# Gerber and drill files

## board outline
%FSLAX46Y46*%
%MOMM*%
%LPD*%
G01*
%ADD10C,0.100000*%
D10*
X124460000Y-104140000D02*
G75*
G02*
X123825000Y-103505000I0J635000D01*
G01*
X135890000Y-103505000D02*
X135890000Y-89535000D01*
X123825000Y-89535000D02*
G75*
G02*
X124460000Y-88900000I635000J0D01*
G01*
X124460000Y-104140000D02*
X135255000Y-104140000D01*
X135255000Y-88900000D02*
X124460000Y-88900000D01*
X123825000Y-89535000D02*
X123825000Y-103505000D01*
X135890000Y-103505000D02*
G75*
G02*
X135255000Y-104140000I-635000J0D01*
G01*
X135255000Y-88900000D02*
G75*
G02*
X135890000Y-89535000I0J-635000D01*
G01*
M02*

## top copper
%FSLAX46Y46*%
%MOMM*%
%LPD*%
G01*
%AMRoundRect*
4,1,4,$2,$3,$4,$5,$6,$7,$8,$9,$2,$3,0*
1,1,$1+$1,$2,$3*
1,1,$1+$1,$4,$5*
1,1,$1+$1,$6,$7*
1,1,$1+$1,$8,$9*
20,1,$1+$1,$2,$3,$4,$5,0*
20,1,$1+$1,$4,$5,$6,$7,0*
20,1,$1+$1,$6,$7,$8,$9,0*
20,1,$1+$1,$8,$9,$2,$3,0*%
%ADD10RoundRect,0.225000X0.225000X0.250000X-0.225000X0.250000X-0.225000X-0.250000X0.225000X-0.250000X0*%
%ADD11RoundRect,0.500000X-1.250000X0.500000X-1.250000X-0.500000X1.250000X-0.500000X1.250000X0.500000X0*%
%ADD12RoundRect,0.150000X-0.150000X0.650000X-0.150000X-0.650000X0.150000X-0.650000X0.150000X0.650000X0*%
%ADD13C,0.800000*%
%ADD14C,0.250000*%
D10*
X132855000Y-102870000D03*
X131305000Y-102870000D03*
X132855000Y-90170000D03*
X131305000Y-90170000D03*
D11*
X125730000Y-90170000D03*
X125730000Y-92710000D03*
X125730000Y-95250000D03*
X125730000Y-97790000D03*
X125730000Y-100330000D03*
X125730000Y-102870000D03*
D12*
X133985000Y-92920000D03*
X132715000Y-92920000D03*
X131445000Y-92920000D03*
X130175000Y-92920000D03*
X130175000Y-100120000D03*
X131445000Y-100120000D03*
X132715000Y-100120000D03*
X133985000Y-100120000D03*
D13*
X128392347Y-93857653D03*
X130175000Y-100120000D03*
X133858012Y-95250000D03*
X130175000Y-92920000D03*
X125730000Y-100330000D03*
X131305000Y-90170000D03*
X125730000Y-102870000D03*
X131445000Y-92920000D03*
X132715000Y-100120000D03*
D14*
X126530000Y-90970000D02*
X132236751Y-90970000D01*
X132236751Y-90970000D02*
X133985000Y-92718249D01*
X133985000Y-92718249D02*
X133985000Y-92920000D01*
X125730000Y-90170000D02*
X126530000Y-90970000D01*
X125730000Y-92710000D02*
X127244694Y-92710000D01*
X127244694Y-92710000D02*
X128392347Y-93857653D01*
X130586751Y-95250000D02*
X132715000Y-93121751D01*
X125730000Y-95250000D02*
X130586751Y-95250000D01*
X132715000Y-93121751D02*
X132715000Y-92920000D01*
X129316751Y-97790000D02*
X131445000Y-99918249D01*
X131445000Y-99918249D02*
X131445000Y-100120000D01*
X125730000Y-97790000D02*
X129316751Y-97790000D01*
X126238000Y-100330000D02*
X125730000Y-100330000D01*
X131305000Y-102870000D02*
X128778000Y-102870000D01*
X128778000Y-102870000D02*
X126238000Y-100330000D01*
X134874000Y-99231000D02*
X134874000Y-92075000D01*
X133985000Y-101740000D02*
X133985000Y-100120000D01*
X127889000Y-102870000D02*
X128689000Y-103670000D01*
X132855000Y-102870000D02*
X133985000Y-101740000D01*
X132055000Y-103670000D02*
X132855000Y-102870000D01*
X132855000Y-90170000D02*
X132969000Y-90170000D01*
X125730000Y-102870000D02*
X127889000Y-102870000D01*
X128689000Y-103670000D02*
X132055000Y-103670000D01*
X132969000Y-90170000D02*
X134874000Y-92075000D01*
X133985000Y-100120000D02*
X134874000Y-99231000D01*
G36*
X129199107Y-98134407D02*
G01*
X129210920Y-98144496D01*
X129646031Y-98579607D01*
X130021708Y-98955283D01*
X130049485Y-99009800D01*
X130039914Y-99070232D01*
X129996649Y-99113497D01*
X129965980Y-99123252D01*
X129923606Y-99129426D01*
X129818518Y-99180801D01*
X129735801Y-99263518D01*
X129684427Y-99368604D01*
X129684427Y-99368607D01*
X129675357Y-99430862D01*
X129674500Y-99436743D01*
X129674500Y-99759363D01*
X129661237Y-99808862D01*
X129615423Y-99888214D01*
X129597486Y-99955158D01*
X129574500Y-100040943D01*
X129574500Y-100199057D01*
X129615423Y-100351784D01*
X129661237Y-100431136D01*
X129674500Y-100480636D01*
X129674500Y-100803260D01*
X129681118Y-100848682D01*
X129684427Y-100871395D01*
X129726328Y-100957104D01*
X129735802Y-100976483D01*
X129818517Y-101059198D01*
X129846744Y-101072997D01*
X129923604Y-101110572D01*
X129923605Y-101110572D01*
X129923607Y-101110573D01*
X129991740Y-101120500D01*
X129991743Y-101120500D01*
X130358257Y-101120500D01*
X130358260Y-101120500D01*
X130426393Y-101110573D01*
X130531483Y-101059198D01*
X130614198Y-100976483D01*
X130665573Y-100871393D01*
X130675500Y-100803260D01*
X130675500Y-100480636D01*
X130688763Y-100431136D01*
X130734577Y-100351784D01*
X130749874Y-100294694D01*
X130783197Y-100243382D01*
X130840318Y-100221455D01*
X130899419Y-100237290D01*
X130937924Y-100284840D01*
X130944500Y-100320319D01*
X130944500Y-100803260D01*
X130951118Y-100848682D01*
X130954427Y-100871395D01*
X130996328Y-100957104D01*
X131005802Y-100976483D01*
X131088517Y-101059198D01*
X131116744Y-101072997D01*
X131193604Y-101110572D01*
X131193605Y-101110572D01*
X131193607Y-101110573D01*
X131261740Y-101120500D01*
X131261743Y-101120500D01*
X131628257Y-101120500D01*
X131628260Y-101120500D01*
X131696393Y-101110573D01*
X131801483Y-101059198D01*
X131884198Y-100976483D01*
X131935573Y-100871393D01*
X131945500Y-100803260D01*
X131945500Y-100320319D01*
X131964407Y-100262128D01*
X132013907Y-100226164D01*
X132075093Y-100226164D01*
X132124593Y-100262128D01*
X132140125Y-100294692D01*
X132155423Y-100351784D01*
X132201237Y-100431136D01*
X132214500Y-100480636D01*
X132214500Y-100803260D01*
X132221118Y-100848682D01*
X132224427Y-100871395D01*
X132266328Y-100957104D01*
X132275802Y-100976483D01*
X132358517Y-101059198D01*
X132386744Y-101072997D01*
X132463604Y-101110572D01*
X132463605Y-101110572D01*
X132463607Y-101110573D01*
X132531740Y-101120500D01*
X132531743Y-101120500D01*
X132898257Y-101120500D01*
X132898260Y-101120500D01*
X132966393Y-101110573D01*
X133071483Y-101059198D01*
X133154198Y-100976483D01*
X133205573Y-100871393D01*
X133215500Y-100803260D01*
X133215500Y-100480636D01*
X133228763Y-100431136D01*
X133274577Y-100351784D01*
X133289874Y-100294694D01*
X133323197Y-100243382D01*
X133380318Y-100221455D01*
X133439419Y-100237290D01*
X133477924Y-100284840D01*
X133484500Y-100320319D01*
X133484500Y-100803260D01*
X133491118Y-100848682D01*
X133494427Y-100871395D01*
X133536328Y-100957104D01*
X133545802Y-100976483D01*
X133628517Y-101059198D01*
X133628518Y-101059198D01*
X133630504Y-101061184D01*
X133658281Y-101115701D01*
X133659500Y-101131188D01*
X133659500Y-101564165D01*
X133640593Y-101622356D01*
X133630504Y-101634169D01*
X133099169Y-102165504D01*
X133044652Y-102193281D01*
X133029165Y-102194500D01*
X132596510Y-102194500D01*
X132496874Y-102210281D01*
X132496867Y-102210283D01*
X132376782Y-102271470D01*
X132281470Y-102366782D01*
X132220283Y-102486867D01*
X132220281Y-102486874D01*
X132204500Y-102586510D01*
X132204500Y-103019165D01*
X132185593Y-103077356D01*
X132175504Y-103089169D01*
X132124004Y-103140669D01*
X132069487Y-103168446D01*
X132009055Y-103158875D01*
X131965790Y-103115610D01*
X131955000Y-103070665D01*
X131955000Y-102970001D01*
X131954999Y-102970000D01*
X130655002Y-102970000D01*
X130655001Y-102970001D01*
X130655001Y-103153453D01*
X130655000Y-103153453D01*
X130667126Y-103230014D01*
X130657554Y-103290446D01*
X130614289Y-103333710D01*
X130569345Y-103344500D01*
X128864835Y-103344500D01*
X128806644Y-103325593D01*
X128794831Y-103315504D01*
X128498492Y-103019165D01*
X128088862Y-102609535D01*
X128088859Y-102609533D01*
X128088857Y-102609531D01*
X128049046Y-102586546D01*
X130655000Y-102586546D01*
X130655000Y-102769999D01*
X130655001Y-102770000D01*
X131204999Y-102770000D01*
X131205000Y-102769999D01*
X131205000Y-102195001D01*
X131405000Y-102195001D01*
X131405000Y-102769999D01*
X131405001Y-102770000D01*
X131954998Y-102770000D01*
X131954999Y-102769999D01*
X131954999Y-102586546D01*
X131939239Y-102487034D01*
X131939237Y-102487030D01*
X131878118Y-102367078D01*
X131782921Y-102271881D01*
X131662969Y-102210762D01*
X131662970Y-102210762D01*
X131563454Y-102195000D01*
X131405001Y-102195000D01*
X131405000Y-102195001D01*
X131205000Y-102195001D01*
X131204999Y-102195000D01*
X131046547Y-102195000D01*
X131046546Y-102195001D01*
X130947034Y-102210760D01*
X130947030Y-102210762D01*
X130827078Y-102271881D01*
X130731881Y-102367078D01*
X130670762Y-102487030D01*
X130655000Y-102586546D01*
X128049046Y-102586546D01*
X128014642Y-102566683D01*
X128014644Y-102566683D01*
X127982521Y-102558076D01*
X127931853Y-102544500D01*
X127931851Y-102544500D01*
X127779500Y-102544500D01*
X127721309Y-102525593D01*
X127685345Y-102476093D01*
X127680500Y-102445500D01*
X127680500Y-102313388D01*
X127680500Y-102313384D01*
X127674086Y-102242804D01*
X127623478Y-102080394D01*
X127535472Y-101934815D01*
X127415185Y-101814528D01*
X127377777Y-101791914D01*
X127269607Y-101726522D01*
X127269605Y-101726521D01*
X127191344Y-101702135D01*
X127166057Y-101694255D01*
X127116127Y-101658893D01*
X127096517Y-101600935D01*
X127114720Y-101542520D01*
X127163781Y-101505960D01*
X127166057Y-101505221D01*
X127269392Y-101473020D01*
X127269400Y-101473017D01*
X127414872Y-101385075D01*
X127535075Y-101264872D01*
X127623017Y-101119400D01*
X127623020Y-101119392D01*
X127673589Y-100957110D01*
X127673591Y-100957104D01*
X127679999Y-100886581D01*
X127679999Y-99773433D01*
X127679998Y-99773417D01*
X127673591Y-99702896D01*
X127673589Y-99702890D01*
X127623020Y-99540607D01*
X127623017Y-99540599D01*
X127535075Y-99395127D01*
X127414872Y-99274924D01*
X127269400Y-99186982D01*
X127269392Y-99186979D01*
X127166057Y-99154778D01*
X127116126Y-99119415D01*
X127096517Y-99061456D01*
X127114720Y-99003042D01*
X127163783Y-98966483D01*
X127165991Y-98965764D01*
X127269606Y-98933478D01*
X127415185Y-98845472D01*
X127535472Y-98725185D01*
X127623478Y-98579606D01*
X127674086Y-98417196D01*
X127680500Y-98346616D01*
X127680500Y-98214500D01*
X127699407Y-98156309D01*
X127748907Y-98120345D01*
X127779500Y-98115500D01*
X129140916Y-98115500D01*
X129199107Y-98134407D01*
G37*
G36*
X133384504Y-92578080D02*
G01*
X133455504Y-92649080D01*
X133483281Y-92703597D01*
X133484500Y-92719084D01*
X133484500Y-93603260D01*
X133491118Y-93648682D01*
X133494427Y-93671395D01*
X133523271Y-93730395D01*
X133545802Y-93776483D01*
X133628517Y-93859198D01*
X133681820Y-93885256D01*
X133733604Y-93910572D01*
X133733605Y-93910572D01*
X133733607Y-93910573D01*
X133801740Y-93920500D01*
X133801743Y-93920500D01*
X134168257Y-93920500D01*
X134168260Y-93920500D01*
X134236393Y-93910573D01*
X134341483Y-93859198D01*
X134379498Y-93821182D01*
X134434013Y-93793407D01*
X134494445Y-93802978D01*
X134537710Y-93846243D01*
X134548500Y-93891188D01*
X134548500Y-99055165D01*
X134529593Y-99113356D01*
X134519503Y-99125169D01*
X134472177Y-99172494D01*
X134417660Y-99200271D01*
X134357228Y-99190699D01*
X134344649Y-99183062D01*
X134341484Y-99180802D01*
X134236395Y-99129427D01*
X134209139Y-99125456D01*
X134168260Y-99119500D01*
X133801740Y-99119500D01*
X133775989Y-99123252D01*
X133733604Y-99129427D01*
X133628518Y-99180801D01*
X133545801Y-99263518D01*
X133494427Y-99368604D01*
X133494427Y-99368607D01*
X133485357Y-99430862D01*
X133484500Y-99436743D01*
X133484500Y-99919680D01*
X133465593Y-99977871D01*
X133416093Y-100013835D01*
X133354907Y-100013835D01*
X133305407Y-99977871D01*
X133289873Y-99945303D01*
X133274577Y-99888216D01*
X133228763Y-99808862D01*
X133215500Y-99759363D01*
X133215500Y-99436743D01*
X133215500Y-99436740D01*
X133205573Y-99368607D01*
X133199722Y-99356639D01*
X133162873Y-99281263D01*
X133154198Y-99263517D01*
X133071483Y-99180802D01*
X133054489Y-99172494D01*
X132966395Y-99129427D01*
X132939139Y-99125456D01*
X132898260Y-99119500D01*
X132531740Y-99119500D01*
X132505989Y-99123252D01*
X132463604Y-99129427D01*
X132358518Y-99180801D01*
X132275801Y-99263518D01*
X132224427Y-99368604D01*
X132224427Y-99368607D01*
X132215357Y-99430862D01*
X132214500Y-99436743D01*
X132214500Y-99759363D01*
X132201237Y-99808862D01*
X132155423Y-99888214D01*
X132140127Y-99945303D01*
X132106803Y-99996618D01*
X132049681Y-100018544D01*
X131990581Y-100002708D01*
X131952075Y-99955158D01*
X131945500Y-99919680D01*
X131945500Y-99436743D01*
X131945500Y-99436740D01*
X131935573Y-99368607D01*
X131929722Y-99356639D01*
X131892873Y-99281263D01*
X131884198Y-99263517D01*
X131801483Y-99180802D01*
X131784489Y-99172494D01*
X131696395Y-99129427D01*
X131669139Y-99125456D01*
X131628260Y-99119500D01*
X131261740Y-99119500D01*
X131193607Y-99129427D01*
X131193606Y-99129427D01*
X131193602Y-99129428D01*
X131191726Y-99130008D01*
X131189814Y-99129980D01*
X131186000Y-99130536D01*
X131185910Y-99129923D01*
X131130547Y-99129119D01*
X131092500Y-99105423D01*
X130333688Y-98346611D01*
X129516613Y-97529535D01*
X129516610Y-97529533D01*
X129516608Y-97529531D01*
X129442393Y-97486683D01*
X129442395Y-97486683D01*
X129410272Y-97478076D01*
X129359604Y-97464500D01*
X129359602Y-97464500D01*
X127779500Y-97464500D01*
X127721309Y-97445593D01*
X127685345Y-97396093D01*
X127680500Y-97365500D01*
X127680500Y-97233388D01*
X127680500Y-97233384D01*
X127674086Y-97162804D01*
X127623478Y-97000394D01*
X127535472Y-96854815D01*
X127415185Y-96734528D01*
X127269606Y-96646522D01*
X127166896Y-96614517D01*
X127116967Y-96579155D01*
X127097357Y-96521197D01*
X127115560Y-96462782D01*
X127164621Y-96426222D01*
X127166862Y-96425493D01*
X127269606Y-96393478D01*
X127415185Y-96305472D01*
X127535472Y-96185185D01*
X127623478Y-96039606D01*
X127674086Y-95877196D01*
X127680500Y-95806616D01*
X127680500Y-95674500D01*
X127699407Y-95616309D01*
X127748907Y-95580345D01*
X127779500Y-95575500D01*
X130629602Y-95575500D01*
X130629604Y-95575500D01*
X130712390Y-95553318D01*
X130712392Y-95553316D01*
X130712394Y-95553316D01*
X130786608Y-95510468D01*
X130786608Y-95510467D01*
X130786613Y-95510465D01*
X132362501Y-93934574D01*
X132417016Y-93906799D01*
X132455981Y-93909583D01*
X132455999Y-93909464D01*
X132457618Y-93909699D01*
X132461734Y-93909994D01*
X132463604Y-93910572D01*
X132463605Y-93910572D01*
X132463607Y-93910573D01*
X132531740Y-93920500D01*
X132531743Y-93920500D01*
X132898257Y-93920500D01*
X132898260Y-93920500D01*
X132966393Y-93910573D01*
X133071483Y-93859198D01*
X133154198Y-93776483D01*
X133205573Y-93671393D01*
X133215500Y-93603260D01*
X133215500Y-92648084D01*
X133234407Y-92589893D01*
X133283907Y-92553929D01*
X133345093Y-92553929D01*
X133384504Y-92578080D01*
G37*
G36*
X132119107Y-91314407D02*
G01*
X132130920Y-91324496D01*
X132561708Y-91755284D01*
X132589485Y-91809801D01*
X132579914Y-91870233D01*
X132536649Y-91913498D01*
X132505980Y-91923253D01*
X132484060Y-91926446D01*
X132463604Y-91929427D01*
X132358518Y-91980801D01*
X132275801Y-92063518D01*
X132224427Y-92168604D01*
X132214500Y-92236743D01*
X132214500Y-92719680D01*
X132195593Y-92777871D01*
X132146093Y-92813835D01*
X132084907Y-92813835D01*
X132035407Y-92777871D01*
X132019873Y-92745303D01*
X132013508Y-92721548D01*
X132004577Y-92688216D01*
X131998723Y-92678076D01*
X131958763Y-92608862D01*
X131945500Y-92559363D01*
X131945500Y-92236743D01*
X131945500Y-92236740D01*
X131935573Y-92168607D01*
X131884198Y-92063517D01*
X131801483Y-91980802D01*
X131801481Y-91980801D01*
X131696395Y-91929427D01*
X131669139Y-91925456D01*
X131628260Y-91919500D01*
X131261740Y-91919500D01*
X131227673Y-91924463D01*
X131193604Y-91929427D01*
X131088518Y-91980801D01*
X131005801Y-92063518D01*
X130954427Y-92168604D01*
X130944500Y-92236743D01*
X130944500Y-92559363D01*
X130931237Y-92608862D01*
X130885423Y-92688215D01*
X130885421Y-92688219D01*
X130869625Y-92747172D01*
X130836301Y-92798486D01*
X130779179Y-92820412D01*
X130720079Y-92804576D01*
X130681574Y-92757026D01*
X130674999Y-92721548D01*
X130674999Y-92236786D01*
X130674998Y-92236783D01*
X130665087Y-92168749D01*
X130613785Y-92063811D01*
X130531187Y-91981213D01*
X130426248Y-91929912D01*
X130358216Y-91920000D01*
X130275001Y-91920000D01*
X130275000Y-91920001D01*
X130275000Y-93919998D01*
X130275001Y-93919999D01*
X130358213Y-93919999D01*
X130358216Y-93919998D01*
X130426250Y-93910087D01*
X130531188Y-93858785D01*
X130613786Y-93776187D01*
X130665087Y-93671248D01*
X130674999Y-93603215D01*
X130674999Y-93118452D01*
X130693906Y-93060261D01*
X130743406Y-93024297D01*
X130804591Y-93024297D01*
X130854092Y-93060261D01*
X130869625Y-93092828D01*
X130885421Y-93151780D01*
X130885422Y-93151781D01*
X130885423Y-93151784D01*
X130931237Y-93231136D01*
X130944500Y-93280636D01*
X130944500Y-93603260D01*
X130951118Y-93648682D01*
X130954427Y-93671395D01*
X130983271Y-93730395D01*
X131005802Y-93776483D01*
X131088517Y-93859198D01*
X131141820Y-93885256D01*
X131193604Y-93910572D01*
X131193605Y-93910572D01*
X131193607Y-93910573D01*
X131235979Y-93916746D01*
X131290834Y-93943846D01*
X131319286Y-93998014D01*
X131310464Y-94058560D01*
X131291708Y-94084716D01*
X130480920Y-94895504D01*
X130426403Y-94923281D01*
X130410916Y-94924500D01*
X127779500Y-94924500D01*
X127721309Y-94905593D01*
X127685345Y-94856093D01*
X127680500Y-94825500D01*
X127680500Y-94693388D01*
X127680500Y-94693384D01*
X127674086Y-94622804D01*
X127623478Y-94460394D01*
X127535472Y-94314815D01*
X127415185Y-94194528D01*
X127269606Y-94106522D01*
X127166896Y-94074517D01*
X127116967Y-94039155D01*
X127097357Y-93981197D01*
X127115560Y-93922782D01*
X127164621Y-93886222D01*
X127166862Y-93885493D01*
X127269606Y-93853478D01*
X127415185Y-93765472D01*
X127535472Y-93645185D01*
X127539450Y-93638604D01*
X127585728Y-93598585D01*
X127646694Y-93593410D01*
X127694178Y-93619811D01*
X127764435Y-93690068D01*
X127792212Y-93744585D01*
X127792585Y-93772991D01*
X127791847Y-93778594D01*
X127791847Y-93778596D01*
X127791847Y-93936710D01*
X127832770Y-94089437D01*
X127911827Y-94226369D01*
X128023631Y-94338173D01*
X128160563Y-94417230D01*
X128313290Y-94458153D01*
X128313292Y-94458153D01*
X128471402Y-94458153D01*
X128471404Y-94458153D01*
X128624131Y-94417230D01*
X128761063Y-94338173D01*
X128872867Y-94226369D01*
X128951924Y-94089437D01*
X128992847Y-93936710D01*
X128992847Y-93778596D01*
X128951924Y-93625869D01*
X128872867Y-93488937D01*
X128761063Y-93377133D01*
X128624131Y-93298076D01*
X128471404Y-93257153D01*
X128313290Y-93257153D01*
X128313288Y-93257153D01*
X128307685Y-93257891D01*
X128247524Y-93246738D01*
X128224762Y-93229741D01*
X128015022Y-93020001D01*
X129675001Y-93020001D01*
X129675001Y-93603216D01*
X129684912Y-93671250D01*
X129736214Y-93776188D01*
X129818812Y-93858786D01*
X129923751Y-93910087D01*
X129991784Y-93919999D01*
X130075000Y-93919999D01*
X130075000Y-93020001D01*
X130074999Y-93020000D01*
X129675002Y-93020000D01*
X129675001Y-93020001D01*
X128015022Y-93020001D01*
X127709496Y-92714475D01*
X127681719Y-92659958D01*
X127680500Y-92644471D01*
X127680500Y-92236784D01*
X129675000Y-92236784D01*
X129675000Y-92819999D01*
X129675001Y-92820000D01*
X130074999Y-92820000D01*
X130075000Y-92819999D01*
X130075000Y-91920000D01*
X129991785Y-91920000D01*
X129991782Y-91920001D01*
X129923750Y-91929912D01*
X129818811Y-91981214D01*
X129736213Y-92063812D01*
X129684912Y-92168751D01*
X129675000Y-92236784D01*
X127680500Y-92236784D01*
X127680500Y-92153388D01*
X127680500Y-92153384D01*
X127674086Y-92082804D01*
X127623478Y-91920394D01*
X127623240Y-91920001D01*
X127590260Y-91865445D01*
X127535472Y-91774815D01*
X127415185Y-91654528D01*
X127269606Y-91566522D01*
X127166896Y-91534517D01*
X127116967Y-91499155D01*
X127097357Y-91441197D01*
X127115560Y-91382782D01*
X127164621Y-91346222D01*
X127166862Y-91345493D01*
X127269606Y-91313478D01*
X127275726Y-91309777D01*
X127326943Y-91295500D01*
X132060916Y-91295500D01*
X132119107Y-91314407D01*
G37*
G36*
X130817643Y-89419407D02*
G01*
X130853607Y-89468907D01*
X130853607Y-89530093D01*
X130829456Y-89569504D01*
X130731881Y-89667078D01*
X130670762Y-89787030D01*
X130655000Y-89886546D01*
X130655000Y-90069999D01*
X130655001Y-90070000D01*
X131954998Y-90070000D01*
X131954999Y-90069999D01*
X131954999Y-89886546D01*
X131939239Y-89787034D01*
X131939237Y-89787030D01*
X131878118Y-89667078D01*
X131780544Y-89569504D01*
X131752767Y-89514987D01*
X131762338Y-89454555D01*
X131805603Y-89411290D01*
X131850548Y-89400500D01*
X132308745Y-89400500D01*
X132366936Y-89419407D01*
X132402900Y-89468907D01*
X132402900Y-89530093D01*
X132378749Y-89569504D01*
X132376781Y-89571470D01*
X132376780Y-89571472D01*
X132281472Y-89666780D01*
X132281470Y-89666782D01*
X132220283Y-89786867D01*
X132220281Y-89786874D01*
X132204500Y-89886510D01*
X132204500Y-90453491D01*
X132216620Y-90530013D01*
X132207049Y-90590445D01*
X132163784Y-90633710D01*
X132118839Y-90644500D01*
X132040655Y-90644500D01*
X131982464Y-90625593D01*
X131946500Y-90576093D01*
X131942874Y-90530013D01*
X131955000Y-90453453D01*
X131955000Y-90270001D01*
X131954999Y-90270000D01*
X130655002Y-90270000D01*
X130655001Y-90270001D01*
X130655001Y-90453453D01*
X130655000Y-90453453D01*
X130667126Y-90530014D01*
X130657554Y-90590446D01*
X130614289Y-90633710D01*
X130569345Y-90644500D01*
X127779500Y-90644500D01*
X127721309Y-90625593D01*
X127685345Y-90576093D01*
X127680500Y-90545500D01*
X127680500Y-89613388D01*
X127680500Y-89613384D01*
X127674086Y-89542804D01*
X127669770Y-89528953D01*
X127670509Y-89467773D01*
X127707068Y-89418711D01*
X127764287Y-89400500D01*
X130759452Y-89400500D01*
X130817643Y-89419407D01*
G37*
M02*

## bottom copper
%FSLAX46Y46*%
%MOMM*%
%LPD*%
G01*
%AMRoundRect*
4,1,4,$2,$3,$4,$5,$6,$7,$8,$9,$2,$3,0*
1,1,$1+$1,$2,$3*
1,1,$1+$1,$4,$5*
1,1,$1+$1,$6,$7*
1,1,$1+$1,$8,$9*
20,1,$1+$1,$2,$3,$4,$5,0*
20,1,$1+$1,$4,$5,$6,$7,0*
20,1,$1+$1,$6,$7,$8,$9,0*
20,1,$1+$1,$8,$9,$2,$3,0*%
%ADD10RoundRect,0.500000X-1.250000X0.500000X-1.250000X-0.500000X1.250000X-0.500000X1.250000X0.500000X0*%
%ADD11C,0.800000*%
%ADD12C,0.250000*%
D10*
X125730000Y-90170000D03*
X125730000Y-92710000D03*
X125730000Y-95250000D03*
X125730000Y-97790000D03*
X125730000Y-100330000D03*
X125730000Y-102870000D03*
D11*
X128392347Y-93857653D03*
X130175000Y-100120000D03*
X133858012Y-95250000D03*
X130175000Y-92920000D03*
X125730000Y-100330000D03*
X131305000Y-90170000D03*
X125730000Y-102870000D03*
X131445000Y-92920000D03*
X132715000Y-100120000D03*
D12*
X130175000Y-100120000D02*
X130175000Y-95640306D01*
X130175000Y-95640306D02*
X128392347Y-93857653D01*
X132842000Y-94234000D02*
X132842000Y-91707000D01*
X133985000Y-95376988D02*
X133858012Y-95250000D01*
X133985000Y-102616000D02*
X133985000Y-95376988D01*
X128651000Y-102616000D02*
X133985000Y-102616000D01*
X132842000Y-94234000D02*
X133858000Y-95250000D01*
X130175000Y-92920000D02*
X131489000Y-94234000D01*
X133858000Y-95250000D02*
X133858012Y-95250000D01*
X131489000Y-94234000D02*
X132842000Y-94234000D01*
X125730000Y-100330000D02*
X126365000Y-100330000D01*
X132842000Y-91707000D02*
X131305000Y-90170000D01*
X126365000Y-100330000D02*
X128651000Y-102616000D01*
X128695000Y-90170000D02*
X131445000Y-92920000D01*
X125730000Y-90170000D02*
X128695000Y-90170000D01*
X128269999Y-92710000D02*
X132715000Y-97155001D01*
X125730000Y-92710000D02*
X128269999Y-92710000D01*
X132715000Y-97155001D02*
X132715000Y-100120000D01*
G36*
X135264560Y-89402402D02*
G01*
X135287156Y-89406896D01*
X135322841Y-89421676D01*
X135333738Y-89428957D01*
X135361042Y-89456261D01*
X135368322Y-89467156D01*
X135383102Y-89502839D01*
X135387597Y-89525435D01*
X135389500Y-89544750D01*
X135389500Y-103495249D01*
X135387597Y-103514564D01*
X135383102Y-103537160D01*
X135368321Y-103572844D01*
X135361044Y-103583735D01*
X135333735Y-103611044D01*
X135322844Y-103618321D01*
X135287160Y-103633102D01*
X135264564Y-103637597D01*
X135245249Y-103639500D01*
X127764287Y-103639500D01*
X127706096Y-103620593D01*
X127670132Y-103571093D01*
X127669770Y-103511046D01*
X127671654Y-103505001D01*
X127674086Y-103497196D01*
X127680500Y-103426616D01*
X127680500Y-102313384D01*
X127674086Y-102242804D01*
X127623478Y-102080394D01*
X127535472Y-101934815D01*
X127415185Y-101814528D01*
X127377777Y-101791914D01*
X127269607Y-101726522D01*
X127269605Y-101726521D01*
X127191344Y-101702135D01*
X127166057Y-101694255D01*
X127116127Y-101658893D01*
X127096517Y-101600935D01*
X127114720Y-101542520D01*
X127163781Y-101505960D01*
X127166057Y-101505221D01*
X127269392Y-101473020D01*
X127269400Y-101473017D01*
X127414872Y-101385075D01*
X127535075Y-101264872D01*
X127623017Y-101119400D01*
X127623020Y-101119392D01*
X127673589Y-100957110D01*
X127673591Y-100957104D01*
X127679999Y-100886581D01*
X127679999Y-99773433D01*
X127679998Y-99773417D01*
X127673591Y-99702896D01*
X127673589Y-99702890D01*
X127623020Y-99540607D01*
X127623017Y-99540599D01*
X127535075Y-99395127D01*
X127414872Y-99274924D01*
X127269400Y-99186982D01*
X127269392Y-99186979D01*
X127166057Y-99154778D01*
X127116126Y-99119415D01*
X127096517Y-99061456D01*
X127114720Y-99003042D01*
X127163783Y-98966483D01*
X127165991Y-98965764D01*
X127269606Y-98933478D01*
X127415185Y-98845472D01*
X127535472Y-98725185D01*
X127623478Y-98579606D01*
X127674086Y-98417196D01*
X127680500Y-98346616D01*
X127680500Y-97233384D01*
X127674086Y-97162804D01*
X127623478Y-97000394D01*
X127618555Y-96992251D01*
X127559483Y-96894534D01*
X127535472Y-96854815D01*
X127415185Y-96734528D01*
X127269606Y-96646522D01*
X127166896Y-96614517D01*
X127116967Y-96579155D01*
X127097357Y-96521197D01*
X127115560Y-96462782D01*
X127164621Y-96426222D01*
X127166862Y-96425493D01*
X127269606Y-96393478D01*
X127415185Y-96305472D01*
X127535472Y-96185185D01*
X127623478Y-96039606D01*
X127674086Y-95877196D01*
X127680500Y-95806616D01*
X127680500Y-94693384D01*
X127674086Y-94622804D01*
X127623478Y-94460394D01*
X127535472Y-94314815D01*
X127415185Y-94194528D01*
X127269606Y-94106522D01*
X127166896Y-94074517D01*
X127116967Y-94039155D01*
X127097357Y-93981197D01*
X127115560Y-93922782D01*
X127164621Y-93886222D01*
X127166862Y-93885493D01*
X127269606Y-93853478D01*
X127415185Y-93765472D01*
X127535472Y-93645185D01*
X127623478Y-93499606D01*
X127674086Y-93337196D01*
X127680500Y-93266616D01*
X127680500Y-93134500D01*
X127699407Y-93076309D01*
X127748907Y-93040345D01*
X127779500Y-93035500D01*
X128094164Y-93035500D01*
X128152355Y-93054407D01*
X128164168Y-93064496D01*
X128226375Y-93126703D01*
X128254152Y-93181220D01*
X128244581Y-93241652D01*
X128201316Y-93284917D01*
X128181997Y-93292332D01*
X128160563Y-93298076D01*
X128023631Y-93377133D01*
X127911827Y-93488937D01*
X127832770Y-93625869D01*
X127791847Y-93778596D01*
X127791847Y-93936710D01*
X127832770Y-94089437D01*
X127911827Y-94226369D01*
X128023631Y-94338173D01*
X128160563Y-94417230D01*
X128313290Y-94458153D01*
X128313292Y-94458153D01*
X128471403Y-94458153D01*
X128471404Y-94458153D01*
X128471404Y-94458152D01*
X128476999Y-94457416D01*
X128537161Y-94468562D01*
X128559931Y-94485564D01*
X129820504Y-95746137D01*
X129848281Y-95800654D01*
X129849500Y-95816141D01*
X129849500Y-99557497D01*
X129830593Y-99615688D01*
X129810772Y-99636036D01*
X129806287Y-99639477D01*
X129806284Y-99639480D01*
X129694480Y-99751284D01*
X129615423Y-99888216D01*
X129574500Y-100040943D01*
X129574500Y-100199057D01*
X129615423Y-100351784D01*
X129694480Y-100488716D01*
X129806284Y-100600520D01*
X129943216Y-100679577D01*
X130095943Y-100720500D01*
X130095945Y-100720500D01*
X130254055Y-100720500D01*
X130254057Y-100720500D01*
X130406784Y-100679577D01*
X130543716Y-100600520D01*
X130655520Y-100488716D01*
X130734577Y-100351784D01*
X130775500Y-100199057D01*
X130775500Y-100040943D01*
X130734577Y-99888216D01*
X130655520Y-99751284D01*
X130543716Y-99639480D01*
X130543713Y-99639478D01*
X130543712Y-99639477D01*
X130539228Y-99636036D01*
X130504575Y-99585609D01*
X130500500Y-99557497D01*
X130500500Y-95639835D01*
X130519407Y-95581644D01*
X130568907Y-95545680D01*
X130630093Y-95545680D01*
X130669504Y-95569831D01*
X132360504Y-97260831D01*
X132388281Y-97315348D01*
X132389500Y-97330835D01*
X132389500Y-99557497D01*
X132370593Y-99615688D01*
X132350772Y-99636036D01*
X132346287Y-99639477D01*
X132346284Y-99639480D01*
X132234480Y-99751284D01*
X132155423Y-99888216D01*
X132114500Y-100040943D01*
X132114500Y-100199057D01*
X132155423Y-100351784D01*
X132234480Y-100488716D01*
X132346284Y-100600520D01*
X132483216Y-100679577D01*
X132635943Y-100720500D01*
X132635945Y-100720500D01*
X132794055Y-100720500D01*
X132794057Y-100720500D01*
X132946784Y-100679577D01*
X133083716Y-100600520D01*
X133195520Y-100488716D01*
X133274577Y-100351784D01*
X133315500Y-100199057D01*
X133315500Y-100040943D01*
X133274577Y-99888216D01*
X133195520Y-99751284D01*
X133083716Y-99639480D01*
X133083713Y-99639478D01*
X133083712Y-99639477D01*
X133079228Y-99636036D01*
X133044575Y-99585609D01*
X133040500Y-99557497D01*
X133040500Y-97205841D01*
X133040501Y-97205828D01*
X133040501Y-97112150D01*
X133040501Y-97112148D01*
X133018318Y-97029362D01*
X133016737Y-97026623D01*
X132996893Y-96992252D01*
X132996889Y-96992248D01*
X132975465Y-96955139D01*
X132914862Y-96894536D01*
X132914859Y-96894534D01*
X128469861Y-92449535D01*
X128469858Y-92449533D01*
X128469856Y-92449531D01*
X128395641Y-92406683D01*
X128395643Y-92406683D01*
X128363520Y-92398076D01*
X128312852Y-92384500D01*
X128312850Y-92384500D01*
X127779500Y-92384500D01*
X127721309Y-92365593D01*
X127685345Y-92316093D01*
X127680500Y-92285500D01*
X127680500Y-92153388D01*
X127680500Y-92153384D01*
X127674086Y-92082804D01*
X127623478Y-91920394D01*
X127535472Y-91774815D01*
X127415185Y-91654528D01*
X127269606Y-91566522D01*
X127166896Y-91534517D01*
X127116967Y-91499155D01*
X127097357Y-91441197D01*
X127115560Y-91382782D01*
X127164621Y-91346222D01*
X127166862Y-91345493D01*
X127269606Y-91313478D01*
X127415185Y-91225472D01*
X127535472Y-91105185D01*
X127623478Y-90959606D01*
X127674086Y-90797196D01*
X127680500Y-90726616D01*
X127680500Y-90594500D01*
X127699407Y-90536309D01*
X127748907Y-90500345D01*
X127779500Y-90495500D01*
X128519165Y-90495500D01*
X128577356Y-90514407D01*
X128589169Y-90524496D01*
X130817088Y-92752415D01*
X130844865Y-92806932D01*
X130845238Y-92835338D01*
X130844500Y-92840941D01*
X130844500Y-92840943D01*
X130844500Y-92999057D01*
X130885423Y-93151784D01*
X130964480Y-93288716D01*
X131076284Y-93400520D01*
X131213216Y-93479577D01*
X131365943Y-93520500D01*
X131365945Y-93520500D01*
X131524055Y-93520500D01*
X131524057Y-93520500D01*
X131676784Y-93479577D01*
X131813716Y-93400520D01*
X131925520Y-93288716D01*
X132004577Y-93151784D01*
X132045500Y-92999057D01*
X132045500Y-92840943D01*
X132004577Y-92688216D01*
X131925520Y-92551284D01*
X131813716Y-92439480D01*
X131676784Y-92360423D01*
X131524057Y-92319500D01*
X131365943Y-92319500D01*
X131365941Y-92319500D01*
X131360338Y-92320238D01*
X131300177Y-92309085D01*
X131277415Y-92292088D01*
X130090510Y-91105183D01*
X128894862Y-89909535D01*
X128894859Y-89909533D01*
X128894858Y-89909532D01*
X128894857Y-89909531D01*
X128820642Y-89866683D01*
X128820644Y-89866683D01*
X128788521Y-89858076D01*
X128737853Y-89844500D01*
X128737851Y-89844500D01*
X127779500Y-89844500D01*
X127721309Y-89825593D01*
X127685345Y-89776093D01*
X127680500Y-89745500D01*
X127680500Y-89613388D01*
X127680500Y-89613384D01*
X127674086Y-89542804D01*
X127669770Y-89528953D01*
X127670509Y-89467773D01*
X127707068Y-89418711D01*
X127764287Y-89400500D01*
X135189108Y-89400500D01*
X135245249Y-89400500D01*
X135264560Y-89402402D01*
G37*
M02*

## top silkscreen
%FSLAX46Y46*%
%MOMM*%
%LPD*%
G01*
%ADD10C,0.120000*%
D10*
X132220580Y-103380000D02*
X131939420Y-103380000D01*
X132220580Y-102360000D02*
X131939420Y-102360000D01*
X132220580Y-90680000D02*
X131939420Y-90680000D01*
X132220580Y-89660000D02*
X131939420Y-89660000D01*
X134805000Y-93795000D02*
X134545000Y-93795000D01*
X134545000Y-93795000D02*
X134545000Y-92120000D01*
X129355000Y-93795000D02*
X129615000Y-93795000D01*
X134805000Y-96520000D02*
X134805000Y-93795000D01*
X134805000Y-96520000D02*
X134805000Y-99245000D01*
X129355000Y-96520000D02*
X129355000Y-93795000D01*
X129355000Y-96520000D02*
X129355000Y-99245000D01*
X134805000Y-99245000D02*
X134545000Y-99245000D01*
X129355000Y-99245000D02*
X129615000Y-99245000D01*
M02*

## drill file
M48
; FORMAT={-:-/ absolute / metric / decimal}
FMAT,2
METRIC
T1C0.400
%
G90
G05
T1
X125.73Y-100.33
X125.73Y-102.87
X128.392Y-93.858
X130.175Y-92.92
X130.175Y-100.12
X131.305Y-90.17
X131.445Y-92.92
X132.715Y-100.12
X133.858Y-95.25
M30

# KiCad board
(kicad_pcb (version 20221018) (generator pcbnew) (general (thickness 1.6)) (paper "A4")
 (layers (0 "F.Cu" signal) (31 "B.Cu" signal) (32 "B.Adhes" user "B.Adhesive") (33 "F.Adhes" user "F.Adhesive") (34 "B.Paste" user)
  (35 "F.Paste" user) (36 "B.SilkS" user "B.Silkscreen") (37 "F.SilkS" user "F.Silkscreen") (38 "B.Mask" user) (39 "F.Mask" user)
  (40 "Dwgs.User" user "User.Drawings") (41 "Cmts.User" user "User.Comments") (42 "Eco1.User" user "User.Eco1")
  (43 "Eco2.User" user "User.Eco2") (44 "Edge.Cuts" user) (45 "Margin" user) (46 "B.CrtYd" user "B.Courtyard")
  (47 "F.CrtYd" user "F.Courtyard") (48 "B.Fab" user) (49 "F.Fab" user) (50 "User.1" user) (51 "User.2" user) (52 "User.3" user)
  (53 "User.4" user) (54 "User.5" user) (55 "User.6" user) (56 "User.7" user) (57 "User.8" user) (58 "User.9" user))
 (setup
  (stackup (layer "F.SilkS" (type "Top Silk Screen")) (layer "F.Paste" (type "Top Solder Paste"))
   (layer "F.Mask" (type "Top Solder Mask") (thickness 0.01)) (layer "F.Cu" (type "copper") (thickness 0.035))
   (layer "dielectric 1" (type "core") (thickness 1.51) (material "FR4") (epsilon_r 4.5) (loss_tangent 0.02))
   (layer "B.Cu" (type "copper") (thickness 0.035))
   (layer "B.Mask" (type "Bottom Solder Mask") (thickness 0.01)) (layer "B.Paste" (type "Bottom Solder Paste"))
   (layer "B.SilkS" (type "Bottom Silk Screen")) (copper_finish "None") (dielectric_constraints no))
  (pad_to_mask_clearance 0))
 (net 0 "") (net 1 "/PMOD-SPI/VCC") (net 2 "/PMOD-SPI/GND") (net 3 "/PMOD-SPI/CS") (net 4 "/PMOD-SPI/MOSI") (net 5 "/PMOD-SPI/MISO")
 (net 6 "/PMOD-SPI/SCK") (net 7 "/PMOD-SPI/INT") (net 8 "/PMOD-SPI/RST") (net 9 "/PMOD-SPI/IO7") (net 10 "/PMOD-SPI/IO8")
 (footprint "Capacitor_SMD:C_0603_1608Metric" (layer "F.Cu") (at 132.08 102.87 180)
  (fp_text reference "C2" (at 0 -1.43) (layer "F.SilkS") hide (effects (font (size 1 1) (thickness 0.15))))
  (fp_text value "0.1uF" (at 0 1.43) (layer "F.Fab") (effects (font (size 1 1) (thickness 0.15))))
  (fp_line (start -0.14058 -0.51) (end 0.14058 -0.51) (stroke (width 0.12) (type solid)) (layer "F.SilkS"))
  (fp_line (start -0.14058 0.51) (end 0.14058 0.51) (stroke (width 0.12) (type solid)) (layer "F.SilkS"))
  (pad "1" smd roundrect (at -0.775 0 180) (size 0.9 0.95) (layers "F.Cu" "F.Paste" "F.Mask") (roundrect_rratio 0.25)
   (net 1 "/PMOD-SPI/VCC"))
  (pad "2" smd roundrect (at 0.775 0 180) (size 0.9 0.95) (layers "F.Cu" "F.Paste" "F.Mask") (roundrect_rratio 0.25) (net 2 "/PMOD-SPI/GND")))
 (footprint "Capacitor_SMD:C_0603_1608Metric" (layer "F.Cu") (at 132.08 90.17 180)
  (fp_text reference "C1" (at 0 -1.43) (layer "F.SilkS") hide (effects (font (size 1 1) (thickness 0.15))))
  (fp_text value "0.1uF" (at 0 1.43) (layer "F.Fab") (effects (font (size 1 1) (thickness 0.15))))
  (fp_line (start -0.14058 -0.51) (end 0.14058 -0.51) (stroke (width 0.12) (type solid)) (layer "F.SilkS"))
  (fp_line (start -0.14058 0.51) (end 0.14058 0.51) (stroke (width 0.12) (type solid)) (layer "F.SilkS"))
  (pad "1" smd roundrect (at -0.775 0 180) (size 0.9 0.95) (layers "F.Cu" "F.Paste" "F.Mask") (roundrect_rratio 0.25)
   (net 1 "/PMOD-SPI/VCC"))
  (pad "2" smd roundrect (at 0.775 0 180) (size 0.9 0.95) (layers "F.Cu" "F.Paste" "F.Mask") (roundrect_rratio 0.25) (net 2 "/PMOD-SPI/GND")))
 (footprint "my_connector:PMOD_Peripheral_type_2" (layer "F.Cu") (at 125.73 96.52 -90)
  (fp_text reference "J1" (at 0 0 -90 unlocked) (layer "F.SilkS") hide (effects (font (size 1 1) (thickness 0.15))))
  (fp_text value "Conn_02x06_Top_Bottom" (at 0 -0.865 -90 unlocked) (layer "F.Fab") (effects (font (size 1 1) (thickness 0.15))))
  (pad "1" smd roundrect (at -6.35 0 270) (size 2 3.5) (layers "F.Cu" "F.Paste" "F.Mask") (roundrect_rratio 0.25) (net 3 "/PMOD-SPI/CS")
   (thermal_bridge_angle 45))
  (pad "2" smd roundrect (at -3.81 0 270) (size 2 3.5) (layers "F.Cu" "F.Paste" "F.Mask") (roundrect_rratio 0.25) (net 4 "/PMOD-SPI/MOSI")
   (thermal_bridge_angle 45))
  (pad "3" smd roundrect (at -1.27 0 270) (size 2 3.5) (layers "F.Cu" "F.Paste" "F.Mask") (roundrect_rratio 0.25) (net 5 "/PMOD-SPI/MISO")
   (thermal_bridge_angle 45))
  (pad "4" smd roundrect (at 1.27 0 270) (size 2 3.5) (layers "F.Cu" "F.Paste" "F.Mask") (roundrect_rratio 0.25) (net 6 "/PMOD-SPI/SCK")
   (thermal_bridge_angle 45))
  (pad "5" smd roundrect (at 3.81 0 270) (size 2 3.5) (layers "F.Cu" "F.Paste" "F.Mask") (roundrect_rratio 0.25) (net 2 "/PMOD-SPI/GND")
   (thermal_bridge_angle 45))
  (pad "6" smd roundrect (at 6.35 0 270) (size 2 3.5) (layers "F.Cu" "F.Paste" "F.Mask") (roundrect_rratio 0.25) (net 1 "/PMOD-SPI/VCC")
   (thermal_bridge_angle 45))
  (pad "7" smd roundrect (at -6.35 0 270) (size 2 3.5) (layers "B.Cu" "B.Paste" "B.Mask") (roundrect_rratio 0.25) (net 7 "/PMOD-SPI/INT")
   (thermal_bridge_angle 45))
  (pad "8" smd roundrect (at -3.81 0 270) (size 2 3.5) (layers "B.Cu" "B.Paste" "B.Mask") (roundrect_rratio 0.25) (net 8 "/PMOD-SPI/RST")
   (thermal_bridge_angle 45))
  (pad "9" smd roundrect (at -1.27 0 270) (size 2 3.5) (layers "B.Cu" "B.Paste" "B.Mask") (roundrect_rratio 0.25) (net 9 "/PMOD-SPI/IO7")
   (thermal_bridge_angle 45))
  (pad "10" smd roundrect (at 1.27 0 270) (size 2 3.5) (layers "B.Cu" "B.Paste" "B.Mask") (roundrect_rratio 0.25) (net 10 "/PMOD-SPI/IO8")
   (thermal_bridge_angle 45))
  (pad "11" smd roundrect (at 3.81 0 270) (size 2 3.5) (layers "B.Cu" "B.Paste" "B.Mask") (roundrect_rratio 0.25) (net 2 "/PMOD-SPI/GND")
   (thermal_bridge_angle 45))
  (pad "12" smd roundrect (at 6.35 0 270) (size 2 3.5) (layers "B.Cu" "B.Paste" "B.Mask") (roundrect_rratio 0.25) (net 1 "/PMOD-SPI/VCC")
   (thermal_bridge_angle 45)))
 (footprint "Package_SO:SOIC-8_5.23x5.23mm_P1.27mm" (layer "F.Cu") (at 132.08 96.52 -90)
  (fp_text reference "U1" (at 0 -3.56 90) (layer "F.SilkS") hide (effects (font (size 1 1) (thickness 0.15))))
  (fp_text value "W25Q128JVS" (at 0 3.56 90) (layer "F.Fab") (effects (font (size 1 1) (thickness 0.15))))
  (fp_line (start -2.725 -2.725) (end -2.725 -2.465) (stroke (width 0.12) (type solid)) (layer "F.SilkS"))
  (fp_line (start -2.725 -2.465) (end -4.4 -2.465) (stroke (width 0.12) (type solid)) (layer "F.SilkS"))
  (fp_line (start -2.725 2.725) (end -2.725 2.465) (stroke (width 0.12) (type solid)) (layer "F.SilkS"))
  (fp_line (start 0 -2.725) (end -2.725 -2.725) (stroke (width 0.12) (type solid)) (layer "F.SilkS"))
  (fp_line (start 0 -2.725) (end 2.725 -2.725) (stroke (width 0.12) (type solid)) (layer "F.SilkS"))
  (fp_line (start 0 2.725) (end -2.725 2.725) (stroke (width 0.12) (type solid)) (layer "F.SilkS"))
  (fp_line (start 0 2.725) (end 2.725 2.725) (stroke (width 0.12) (type solid)) (layer "F.SilkS"))
  (fp_line (start 2.725 -2.725) (end 2.725 -2.465) (stroke (width 0.12) (type solid)) (layer "F.SilkS"))
  (fp_line (start 2.725 2.725) (end 2.725 2.465) (stroke (width 0.12) (type solid)) (layer "F.SilkS"))
  (pad "1" smd roundrect (at -3.6 -1.905 270) (size 1.6 0.6) (layers "F.Cu" "F.Paste" "F.Mask") (roundrect_rratio 0.25)
   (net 3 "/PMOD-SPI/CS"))
  (pad "2" smd roundrect (at -3.6 -0.635 270) (size 1.6 0.6) (layers "F.Cu" "F.Paste" "F.Mask") (roundrect_rratio 0.25)
   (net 5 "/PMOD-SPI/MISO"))
  (pad "3" smd roundrect (at -3.6 0.635 270) (size 1.6 0.6) (layers "F.Cu" "F.Paste" "F.Mask") (roundrect_rratio 0.25)
   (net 7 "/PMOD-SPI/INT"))
  (pad "4" smd roundrect (at -3.6 1.905 270) (size 1.6 0.6) (layers "F.Cu" "F.Paste" "F.Mask") (roundrect_rratio 0.25)
   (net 2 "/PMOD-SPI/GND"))
  (pad "5" smd roundrect (at 3.6 1.905 270) (size 1.6 0.6) (layers "F.Cu" "F.Paste" "F.Mask") (roundrect_rratio 0.25)
   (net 4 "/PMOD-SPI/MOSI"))
  (pad "6" smd roundrect (at 3.6 0.635 270) (size 1.6 0.6) (layers "F.Cu" "F.Paste" "F.Mask") (roundrect_rratio 0.25)
   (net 6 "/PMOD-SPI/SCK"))
  (pad "7" smd roundrect (at 3.6 -0.635 270) (size 1.6 0.6) (layers "F.Cu" "F.Paste" "F.Mask") (roundrect_rratio 0.25)
   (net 8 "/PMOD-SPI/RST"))
  (pad "8" smd roundrect (at 3.6 -1.905 270) (size 1.6 0.6) (layers "F.Cu" "F.Paste" "F.Mask") (roundrect_rratio 0.25)
   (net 1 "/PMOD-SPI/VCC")))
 (gr_arc (start 124.46 104.14) (mid 124.010987 103.954013) (end 123.825 103.505) (stroke (width 0.1) (type default)) (layer "Edge.Cuts"))
 (gr_line (start 135.89 103.505) (end 135.89 89.535) (stroke (width 0.1) (type default)) (layer "Edge.Cuts"))
 (gr_arc (start 123.825 89.535) (mid 124.010987 89.085987) (end 124.46 88.9) (stroke (width 0.1) (type default)) (layer "Edge.Cuts"))
 (gr_line (start 124.46 104.14) (end 135.255 104.14) (stroke (width 0.1) (type default)) (layer "Edge.Cuts"))
 (gr_line (start 135.255 88.9) (end 124.46 88.9) (stroke (width 0.1) (type default)) (layer "Edge.Cuts"))
 (gr_line (start 123.825 89.535) (end 123.825 103.505) (stroke (width 0.1) (type default)) (layer "Edge.Cuts"))
 (gr_arc (start 135.89 103.505) (mid 135.704013 103.954013) (end 135.255 104.14) (stroke (width 0.1) (type default)) (layer "Edge.Cuts"))
 (gr_arc (start 135.255 88.9) (mid 135.704013 89.085987) (end 135.89 89.535) (stroke (width 0.1) (type default)) (layer "Edge.Cuts"))
 (segment (start 126.53 90.97) (end 132.236751 90.97) (width 0.25) (layer "F.Cu") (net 3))
 (segment (start 132.236751 90.97) (end 133.985 92.718249) (width 0.25) (layer "F.Cu") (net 3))
 (segment (start 133.985 92.718249) (end 133.985 92.92) (width 0.25) (layer "F.Cu") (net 3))
 (segment (start 125.73 90.17) (end 126.53 90.97) (width 0.25) (layer "F.Cu") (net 3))
 (segment (start 125.73 92.71) (end 127.244694 92.71) (width 0.25) (layer "F.Cu") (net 4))
 (segment (start 127.244694 92.71) (end 128.392347 93.857653) (width 0.25) (layer "F.Cu") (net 4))
 (via (at 128.392347 93.857653) (size 0.8) (drill 0.4) (layers "F.Cu" "B.Cu") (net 4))
 (via (at 130.175 100.12) (size 0.8) (drill 0.4) (layers "F.Cu" "B.Cu") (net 4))
 (segment (start 130.175 100.12) (end 130.175 95.640306) (width 0.25) (layer "B.Cu") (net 4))
 (segment (start 130.175 95.640306) (end 128.392347 93.857653) (width 0.25) (layer "B.Cu") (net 4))
 (segment (start 130.586751 95.25) (end 132.715 93.121751) (width 0.25) (layer "F.Cu") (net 5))
 (segment (start 125.73 95.25) (end 130.586751 95.25) (width 0.25) (layer "F.Cu") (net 5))
 (segment (start 132.715 93.121751) (end 132.715 92.92) (width 0.25) (layer "F.Cu") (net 5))
 (segment (start 129.316751 97.79) (end 131.445 99.918249) (width 0.25) (layer "F.Cu") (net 6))
 (segment (start 131.445 99.918249) (end 131.445 100.12) (width 0.25) (layer "F.Cu") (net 6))
 (segment (start 125.73 97.79) (end 129.316751 97.79) (width 0.25) (layer "F.Cu") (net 6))
 (segment (start 126.238 100.33) (end 125.73 100.33) (width 0.25) (layer "F.Cu") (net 2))
 (segment (start 131.305 102.87) (end 128.778 102.87) (width 0.25) (layer "F.Cu") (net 2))
 (segment (start 128.778 102.87) (end 126.238 100.33) (width 0.25) (layer "F.Cu") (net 2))
 (via (at 133.858012 95.25) (size 0.8) (drill 0.4) (layers "F.Cu" "B.Cu") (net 2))
 (via (at 130.175 92.92) (size 0.8) (drill 0.4) (layers "F.Cu" "B.Cu") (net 2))
 (via (at 125.73 100.33) (size 0.8) (drill 0.4) (layers "F.Cu" "B.Cu") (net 2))
 (via (at 131.305 90.17) (size 0.8) (drill 0.4) (layers "F.Cu" "B.Cu") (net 2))
 (segment (start 132.842 94.234) (end 132.842 91.707) (width 0.25) (layer "B.Cu") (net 2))
 (segment (start 133.985 95.376988) (end 133.858012 95.25) (width 0.25) (layer "B.Cu") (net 2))
 (segment (start 133.985 102.616) (end 133.985 95.376988) (width 0.25) (layer "B.Cu") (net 2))
 (segment (start 128.651 102.616) (end 133.985 102.616) (width 0.25) (layer "B.Cu") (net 2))
 (segment (start 132.842 94.234) (end 133.858 95.25) (width 0.25) (layer "B.Cu") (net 2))
 (segment (start 130.175 92.92) (end 131.489 94.234) (width 0.25) (layer "B.Cu") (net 2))
 (segment (start 133.858 95.25) (end 133.858012 95.25) (width 0.25) (layer "B.Cu") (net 2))
 (segment (start 131.489 94.234) (end 132.842 94.234) (width 0.25) (layer "B.Cu") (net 2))
 (segment (start 125.73 100.33) (end 126.365 100.33) (width 0.25) (layer "B.Cu") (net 2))
 (segment (start 132.842 91.707) (end 131.305 90.17) (width 0.25) (layer "B.Cu") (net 2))
 (segment (start 126.365 100.33) (end 128.651 102.616) (width 0.25) (layer "B.Cu") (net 2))
 (segment (start 134.874 99.231) (end 134.874 92.075) (width 0.25) (layer "F.Cu") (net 1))
 (segment (start 133.985 101.74) (end 133.985 100.12) (width 0.25) (layer "F.Cu") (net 1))
 (segment (start 127.889 102.87) (end 128.689 103.67) (width 0.25) (layer "F.Cu") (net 1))
 (segment (start 132.855 102.87) (end 133.985 101.74) (width 0.25) (layer "F.Cu") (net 1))
 (segment (start 132.055 103.67) (end 132.855 102.87) (width 0.25) (layer "F.Cu") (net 1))
 (segment (start 132.855 90.17) (end 132.969 90.17) (width 0.25) (layer "F.Cu") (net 1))
 (segment (start 125.73 102.87) (end 127.889 102.87) (width 0.25) (layer "F.Cu") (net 1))
 (segment (start 128.689 103.67) (end 132.055 103.67) (width 0.25) (layer "F.Cu") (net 1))
 (segment (start 132.969 90.17) (end 134.874 92.075) (width 0.25) (layer "F.Cu") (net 1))
 (segment (start 133.985 100.12) (end 134.874 99.231) (width 0.25) (layer "F.Cu") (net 1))
 (via (at 125.73 102.87) (size 0.8) (drill 0.4) (layers "F.Cu" "B.Cu") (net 1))
 (via (at 131.445 92.92) (size 0.8) (drill 0.4) (layers "F.Cu" "B.Cu") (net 7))
 (segment (start 128.695 90.17) (end 131.445 92.92) (width 0.25) (layer "B.Cu") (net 7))
 (segment (start 125.73 90.17) (end 128.695 90.17) (width 0.25) (layer "B.Cu") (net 7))
 (via (at 132.715 100.12) (size 0.8) (drill 0.4) (layers "F.Cu" "B.Cu") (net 8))
 (segment (start 128.269999 92.71) (end 132.715 97.155001) (width 0.25) (layer "B.Cu") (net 8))
 (segment (start 125.73 92.71) (end 128.269999 92.71) (width 0.25) (layer "B.Cu") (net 8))
 (segment (start 132.715 97.155001) (end 132.715 100.12) (width 0.25) (layer "B.Cu") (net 8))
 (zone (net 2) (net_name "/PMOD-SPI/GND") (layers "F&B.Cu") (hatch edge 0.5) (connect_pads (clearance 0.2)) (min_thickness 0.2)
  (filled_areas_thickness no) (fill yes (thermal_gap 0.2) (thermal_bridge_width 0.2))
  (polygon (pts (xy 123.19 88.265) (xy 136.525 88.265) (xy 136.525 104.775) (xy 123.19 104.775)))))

